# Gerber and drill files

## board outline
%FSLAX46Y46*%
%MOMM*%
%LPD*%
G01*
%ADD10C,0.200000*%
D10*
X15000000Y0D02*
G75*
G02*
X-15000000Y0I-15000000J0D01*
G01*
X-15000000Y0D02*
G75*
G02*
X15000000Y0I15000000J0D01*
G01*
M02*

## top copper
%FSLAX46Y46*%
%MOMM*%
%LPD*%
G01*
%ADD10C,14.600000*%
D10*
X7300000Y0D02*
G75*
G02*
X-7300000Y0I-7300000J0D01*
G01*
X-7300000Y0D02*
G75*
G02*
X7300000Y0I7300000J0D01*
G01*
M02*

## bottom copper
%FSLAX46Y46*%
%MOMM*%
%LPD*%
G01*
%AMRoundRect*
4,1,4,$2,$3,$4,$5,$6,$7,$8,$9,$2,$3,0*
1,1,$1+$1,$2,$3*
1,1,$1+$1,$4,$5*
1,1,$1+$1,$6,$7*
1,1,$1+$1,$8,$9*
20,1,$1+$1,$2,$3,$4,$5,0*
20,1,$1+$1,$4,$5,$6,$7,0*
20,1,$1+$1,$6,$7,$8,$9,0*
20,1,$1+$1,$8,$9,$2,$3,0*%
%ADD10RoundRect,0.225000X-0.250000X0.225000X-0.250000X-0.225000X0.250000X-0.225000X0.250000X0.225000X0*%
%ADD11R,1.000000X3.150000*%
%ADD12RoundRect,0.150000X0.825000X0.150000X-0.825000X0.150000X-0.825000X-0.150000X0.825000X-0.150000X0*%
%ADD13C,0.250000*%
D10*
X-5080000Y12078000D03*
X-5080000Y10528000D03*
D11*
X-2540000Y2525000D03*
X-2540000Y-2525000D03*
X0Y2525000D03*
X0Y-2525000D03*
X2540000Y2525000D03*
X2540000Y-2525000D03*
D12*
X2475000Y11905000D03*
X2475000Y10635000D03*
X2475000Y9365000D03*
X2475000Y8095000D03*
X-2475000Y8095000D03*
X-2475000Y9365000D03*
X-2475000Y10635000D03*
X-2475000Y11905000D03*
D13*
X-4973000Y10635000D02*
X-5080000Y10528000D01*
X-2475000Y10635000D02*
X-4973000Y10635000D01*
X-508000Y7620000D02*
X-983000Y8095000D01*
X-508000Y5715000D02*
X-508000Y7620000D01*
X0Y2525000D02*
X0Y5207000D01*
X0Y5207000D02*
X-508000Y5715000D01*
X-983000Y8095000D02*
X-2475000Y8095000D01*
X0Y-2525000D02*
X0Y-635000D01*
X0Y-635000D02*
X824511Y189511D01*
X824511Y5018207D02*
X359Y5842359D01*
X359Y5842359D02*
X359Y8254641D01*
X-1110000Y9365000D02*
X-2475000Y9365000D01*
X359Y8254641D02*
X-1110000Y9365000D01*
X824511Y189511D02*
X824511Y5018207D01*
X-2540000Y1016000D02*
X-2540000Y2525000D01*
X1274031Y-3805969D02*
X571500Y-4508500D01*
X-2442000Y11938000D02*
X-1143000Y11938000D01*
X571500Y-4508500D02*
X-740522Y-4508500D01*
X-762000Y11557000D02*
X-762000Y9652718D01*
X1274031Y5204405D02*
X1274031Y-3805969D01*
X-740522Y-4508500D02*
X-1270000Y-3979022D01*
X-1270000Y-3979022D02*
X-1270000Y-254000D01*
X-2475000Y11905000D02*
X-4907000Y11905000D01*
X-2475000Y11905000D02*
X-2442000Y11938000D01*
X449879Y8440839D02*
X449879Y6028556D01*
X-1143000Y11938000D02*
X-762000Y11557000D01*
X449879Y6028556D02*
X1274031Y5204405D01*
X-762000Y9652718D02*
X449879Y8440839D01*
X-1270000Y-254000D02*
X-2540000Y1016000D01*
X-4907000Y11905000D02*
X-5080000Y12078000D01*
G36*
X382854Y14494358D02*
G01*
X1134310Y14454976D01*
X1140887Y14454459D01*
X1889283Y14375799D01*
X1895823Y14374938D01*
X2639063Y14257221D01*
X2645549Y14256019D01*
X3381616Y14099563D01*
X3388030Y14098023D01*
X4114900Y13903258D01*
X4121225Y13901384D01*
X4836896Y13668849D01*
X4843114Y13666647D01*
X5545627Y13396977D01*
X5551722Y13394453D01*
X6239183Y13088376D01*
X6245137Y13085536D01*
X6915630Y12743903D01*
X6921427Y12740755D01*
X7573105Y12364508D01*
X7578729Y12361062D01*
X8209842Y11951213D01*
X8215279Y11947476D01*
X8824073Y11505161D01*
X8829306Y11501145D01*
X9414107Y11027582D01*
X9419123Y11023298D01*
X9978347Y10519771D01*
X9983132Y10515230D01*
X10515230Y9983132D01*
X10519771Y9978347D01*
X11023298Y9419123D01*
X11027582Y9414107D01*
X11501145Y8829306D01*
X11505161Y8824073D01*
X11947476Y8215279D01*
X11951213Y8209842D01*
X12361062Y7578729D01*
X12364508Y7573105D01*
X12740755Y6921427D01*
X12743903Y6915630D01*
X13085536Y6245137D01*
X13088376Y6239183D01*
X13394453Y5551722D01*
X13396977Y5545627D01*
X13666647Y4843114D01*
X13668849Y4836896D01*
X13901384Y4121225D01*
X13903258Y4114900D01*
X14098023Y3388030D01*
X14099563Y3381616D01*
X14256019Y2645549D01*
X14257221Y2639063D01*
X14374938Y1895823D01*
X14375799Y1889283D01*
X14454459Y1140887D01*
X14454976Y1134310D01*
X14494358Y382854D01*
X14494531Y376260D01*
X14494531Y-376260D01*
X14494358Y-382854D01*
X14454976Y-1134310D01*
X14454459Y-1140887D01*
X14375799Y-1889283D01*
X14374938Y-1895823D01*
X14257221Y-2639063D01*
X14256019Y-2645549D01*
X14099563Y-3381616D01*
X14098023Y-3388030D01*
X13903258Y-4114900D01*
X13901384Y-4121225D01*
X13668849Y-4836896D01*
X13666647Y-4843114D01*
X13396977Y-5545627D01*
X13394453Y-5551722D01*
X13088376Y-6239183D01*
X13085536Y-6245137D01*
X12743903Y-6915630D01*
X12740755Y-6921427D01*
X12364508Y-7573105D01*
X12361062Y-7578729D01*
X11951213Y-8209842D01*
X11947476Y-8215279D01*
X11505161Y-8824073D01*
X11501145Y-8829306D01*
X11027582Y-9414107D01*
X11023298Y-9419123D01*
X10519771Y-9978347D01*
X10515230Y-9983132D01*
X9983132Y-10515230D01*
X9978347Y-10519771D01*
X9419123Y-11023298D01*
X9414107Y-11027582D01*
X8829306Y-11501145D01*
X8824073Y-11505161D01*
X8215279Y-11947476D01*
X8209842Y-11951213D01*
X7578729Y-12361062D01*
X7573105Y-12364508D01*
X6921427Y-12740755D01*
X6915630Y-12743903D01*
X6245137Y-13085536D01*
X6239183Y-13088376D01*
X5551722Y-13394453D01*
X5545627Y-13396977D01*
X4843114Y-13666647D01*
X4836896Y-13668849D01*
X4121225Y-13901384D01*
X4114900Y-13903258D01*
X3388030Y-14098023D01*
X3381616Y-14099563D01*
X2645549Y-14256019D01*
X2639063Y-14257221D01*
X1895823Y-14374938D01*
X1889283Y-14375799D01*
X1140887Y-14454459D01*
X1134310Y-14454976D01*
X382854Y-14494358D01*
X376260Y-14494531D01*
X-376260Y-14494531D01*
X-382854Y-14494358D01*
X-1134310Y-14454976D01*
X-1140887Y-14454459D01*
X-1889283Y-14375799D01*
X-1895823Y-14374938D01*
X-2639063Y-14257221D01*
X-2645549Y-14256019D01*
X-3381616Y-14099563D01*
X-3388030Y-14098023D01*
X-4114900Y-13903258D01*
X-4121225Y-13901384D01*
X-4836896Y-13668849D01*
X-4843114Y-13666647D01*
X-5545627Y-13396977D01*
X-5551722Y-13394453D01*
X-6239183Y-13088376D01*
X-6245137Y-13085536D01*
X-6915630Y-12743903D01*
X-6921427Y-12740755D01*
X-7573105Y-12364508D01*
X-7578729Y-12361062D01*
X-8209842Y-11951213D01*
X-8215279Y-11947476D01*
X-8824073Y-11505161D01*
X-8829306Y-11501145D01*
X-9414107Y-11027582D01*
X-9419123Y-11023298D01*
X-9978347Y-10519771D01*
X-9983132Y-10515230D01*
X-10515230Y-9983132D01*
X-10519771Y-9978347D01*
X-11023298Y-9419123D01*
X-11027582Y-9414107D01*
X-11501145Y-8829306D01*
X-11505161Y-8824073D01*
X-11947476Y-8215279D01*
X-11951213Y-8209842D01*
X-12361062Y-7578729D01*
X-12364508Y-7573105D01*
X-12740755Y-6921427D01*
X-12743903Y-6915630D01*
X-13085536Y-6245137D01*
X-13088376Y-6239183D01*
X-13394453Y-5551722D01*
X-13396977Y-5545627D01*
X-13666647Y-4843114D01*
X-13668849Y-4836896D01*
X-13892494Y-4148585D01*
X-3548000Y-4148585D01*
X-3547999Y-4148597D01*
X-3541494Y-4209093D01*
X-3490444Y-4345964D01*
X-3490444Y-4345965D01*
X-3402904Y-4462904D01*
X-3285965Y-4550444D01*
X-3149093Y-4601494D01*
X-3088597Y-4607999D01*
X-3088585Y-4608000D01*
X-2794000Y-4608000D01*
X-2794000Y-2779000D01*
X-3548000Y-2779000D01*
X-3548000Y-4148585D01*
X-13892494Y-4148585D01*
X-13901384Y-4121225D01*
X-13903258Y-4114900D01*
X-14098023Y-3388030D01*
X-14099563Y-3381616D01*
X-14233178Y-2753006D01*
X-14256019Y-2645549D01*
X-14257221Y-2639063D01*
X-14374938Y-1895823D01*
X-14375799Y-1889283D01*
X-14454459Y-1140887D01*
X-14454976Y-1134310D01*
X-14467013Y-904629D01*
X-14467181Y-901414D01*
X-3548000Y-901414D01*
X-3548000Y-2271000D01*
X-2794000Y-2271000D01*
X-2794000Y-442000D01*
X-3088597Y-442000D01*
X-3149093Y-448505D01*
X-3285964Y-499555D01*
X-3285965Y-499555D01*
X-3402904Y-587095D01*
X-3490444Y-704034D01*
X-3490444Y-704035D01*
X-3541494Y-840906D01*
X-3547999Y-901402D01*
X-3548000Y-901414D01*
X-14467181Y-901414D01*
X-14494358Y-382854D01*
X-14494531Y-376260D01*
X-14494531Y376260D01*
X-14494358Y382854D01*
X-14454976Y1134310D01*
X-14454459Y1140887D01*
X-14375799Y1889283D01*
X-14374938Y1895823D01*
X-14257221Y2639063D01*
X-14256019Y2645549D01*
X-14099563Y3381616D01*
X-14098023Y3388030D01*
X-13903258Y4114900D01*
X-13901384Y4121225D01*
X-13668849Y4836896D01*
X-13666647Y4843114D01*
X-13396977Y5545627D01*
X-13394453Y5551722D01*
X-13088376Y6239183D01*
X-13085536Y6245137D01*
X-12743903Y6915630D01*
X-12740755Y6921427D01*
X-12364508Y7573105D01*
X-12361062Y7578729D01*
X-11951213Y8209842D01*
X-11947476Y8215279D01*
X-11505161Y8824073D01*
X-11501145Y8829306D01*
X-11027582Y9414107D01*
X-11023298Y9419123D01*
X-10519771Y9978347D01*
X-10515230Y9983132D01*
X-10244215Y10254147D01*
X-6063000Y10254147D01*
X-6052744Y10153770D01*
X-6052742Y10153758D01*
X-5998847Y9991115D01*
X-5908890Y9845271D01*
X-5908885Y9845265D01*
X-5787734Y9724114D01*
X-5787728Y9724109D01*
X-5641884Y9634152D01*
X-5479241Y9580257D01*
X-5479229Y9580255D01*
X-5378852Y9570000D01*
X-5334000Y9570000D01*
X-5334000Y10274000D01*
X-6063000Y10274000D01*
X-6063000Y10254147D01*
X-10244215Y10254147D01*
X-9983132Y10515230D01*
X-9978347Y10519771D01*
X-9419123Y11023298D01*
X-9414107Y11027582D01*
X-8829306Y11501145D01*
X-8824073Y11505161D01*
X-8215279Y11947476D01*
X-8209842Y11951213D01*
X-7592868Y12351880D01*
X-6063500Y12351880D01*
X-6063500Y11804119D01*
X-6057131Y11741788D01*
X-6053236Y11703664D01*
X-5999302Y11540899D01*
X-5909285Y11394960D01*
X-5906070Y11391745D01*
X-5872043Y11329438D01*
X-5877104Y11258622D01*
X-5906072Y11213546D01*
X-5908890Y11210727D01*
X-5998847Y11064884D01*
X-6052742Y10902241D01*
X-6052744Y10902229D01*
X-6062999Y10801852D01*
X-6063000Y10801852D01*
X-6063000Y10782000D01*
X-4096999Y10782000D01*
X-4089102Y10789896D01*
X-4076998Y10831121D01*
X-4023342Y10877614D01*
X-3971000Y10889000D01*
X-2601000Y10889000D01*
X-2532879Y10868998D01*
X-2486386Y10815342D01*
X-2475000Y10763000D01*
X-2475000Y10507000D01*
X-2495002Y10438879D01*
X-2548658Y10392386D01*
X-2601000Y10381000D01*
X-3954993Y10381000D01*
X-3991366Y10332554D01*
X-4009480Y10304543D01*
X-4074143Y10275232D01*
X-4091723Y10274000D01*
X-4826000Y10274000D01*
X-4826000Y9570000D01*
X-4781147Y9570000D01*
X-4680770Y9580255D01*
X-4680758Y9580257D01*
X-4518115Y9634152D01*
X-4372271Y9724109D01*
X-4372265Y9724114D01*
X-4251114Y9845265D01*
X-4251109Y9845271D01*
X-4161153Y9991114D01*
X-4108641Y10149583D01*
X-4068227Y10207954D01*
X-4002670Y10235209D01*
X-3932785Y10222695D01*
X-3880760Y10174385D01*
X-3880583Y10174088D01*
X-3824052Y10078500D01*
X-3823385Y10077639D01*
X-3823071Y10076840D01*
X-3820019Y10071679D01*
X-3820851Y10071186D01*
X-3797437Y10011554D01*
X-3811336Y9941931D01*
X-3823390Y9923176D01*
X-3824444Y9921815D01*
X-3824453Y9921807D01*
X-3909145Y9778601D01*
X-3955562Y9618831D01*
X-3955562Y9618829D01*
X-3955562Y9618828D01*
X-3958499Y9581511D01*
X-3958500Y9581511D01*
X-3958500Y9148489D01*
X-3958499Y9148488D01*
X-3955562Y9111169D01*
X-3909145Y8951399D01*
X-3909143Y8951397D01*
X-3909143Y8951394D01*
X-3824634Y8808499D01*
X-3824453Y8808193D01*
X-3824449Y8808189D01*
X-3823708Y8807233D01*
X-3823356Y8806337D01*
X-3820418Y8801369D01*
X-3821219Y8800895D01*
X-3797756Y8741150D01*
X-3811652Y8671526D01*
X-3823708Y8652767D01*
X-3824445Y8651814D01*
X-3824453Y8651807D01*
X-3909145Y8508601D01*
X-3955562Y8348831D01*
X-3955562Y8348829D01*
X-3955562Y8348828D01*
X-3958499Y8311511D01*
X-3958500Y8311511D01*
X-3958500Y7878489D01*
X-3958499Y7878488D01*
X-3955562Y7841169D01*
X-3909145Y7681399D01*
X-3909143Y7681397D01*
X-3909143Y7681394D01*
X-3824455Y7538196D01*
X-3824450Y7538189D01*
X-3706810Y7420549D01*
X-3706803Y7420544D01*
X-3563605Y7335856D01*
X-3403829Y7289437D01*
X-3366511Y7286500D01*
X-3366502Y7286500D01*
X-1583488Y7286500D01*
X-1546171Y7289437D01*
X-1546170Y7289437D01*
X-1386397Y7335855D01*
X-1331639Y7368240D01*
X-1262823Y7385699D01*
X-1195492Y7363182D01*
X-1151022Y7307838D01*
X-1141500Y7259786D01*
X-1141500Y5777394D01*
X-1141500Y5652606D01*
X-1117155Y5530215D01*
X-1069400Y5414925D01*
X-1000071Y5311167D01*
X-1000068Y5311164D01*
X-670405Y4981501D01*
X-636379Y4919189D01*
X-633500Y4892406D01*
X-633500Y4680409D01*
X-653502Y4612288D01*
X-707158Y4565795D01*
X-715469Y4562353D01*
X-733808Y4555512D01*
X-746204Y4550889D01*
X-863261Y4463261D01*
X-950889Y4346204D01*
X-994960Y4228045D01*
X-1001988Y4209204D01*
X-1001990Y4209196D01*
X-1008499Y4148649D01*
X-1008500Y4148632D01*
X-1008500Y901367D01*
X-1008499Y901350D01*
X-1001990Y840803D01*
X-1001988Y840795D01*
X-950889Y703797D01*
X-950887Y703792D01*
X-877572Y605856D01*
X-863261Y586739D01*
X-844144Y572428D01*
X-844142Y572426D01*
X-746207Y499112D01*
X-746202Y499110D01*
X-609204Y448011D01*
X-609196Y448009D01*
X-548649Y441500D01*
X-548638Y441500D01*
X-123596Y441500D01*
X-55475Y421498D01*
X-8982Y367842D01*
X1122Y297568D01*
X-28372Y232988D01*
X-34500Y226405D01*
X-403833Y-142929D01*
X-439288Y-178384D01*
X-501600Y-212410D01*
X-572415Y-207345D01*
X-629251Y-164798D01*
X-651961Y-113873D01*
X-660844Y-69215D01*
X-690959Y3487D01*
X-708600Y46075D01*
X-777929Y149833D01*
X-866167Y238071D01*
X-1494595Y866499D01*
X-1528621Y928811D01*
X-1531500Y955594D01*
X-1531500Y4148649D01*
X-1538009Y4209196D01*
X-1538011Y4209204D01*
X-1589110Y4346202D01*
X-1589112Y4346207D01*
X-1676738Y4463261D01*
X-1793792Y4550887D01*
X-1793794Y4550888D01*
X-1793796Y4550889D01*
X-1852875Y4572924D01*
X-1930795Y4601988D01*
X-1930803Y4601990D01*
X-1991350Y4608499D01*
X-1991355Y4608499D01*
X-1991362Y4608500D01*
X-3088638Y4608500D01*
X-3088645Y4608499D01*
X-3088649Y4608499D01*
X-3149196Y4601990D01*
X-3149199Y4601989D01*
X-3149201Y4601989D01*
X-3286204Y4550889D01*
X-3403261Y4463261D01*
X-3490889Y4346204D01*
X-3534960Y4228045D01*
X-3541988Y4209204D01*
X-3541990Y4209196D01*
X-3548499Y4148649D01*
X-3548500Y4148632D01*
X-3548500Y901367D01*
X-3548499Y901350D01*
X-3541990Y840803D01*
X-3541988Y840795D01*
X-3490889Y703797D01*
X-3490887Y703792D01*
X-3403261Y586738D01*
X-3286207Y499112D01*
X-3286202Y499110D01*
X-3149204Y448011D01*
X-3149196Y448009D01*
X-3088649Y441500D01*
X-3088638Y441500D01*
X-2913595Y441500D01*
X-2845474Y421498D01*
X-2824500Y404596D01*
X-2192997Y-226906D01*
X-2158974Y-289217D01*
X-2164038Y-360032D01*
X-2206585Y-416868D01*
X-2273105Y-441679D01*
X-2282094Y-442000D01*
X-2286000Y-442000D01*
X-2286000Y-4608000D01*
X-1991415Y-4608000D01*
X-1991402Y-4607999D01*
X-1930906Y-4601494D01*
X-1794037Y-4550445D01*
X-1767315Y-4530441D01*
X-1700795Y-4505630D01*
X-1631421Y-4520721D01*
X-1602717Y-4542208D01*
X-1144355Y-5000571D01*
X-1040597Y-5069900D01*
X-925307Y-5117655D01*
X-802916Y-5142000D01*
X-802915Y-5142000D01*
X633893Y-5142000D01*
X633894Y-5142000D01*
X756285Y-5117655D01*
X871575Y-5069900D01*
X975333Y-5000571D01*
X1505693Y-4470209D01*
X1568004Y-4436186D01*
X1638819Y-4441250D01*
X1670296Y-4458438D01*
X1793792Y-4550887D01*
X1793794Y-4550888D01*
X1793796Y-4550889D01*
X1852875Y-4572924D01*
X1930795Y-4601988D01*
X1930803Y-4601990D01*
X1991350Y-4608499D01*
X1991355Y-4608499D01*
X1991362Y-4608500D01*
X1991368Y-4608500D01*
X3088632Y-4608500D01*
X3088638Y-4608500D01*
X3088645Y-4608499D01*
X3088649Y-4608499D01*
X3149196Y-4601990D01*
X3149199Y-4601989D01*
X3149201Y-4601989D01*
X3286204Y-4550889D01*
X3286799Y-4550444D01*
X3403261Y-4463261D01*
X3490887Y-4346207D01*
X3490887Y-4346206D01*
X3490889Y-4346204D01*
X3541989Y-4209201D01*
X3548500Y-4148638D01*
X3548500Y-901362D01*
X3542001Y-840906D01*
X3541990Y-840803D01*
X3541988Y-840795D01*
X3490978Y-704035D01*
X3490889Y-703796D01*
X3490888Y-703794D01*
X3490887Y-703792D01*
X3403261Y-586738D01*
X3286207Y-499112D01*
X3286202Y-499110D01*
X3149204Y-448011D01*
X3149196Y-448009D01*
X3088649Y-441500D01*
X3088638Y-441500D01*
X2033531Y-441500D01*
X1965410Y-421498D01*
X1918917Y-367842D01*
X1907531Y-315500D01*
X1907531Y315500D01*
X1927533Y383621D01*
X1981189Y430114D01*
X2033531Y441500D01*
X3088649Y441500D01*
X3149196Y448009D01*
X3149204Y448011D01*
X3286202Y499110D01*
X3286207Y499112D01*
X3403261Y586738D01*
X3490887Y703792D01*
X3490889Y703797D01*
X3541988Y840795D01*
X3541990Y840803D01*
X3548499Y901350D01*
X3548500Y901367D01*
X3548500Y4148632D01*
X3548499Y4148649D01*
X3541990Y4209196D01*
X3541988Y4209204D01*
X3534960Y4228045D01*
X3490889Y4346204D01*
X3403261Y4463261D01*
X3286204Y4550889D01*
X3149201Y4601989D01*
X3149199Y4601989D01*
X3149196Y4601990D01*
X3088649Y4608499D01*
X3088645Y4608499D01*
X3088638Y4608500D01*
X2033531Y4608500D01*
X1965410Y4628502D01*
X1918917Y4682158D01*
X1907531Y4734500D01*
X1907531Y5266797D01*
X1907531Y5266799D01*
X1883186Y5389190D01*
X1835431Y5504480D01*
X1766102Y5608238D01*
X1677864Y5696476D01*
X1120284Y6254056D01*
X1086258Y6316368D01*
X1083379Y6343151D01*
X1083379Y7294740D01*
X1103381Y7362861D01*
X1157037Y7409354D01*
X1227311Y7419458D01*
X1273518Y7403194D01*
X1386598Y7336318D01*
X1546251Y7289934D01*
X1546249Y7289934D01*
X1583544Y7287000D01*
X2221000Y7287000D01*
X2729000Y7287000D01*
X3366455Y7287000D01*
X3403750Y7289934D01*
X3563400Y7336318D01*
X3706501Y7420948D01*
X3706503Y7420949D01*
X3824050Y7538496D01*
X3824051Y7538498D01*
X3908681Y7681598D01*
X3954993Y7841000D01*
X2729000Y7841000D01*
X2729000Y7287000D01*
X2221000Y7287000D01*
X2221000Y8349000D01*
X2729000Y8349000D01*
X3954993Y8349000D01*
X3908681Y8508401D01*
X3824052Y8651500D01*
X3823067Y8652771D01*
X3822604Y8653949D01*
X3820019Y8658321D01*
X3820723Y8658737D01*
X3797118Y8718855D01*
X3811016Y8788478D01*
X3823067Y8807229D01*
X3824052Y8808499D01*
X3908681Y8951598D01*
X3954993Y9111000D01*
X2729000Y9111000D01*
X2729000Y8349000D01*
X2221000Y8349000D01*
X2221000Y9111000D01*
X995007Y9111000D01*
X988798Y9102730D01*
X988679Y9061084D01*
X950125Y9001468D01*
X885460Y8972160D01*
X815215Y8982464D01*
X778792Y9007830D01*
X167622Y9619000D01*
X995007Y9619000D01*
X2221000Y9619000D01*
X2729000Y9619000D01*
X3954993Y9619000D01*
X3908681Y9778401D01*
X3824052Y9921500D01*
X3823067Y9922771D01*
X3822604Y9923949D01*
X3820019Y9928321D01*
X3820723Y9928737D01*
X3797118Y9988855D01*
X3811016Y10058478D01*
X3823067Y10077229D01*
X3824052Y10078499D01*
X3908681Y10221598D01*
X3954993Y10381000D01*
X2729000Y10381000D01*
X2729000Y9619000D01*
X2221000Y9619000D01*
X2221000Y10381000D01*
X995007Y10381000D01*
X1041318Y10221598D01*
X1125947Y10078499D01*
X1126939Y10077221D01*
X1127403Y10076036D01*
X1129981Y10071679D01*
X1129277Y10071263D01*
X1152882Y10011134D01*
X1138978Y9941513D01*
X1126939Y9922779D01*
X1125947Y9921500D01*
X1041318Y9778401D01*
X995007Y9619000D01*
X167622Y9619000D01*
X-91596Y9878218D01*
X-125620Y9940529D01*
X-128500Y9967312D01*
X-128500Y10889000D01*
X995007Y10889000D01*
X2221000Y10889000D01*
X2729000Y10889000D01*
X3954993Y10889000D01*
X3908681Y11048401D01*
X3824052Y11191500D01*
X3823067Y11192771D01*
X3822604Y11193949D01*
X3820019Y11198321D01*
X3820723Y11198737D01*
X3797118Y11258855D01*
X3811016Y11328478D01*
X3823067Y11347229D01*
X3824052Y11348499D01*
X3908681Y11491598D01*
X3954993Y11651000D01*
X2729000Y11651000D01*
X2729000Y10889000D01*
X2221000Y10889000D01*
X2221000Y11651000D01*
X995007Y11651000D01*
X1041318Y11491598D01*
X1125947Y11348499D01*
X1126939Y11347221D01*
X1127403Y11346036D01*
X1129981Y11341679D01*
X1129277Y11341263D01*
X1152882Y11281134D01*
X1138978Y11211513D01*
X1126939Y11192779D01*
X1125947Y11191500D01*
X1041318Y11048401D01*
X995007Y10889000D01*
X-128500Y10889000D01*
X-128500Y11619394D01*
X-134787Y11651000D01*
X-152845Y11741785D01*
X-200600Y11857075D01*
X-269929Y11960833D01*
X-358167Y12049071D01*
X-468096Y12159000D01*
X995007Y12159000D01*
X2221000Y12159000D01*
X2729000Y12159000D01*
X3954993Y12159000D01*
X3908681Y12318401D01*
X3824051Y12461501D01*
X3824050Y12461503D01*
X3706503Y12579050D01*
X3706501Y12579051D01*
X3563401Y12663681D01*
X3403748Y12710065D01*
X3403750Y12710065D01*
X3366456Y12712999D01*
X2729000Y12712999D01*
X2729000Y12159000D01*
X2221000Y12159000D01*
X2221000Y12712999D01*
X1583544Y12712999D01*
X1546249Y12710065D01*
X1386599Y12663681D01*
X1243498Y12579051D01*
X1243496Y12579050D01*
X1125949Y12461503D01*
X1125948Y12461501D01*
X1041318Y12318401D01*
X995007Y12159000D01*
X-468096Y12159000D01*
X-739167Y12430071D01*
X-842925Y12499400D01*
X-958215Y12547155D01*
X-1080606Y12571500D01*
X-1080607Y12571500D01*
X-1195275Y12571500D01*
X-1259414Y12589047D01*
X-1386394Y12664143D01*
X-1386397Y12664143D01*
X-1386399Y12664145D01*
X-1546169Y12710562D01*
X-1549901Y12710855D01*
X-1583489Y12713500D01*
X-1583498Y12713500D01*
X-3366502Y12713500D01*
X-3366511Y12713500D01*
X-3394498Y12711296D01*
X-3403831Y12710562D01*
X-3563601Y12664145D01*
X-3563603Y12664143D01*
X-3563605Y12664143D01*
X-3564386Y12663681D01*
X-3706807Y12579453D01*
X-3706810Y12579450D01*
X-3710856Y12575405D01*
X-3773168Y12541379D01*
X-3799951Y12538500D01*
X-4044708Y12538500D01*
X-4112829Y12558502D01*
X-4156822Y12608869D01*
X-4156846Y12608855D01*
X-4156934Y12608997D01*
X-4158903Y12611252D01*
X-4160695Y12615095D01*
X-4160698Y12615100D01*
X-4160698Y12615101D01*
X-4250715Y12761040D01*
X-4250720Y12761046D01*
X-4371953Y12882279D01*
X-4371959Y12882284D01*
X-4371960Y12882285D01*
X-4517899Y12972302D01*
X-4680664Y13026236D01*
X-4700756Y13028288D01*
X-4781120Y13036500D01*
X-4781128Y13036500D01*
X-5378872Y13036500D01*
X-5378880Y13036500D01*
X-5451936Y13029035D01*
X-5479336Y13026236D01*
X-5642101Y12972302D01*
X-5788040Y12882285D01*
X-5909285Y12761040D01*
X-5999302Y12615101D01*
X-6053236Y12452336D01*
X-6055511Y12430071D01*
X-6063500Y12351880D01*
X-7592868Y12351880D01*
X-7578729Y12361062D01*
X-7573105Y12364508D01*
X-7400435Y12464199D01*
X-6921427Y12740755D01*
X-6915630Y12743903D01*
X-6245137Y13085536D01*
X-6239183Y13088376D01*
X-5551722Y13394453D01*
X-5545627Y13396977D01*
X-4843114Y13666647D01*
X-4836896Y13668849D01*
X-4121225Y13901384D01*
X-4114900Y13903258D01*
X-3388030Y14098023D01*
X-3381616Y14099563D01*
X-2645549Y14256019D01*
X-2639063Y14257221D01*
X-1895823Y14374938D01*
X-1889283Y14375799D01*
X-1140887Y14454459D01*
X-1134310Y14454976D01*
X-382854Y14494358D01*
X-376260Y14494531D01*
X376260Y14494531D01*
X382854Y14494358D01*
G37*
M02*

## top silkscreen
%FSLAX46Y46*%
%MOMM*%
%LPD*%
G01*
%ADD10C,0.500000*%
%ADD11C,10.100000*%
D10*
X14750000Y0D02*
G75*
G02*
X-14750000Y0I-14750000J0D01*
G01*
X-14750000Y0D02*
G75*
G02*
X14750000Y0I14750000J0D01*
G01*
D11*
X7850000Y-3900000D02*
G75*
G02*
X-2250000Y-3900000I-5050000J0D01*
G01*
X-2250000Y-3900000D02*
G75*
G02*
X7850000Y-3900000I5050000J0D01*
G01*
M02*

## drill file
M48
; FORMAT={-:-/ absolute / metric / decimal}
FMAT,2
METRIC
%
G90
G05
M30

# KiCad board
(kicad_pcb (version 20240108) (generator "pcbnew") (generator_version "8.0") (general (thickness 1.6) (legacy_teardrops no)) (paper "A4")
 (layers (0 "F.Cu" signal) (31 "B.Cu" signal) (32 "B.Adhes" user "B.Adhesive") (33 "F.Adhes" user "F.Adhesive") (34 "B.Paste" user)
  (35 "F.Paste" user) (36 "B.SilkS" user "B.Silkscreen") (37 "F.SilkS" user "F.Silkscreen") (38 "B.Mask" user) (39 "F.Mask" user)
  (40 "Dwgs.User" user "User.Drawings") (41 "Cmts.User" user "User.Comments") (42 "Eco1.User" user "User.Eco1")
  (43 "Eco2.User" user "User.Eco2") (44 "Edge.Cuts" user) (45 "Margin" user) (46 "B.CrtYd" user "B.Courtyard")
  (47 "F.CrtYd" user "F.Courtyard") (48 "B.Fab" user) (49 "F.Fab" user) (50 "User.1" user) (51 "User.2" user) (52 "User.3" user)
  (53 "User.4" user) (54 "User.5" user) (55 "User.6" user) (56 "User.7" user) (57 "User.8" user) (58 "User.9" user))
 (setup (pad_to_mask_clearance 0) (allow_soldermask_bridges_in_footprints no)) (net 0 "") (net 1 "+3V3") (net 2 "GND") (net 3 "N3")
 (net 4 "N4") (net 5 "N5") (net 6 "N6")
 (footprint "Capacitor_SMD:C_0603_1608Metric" (layer "B.Cu") (at -5.08 -11.303 -90)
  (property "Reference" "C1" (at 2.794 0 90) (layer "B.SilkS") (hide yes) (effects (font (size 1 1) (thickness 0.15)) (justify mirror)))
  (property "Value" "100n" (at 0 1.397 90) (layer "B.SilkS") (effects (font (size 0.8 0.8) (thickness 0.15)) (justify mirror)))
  (pad "1" smd roundrect (at -0.775 0 270) (size 0.9 0.95) (layers "B.Cu" "B.Paste" "B.Mask") (roundrect_rratio 0.25) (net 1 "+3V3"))
  (pad "2" smd roundrect (at 0.775 0 270) (size 0.9 0.95) (layers "B.Cu" "B.Paste" "B.Mask") (roundrect_rratio 0.25) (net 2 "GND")))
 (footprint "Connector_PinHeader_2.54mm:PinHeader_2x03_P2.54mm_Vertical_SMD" (layer "B.Cu") (at 0 0 -90)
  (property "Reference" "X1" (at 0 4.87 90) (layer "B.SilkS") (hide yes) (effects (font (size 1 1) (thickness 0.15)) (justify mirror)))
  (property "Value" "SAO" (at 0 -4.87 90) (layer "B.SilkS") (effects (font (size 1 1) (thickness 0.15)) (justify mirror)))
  (pad "1" smd rect (at -2.525 2.54 270) (size 3.15 1) (layers "B.Cu" "B.Paste" "B.Mask") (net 1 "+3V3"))
  (pad "2" smd rect (at 2.525 2.54 270) (size 3.15 1) (layers "B.Cu" "B.Paste" "B.Mask") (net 2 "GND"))
  (pad "3" smd rect (at -2.525 0 270) (size 3.15 1) (layers "B.Cu" "B.Paste" "B.Mask") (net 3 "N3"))
  (pad "4" smd rect (at 2.525 0 270) (size 3.15 1) (layers "B.Cu" "B.Paste" "B.Mask") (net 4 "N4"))
  (pad "5" smd rect (at -2.525 -2.54 270) (size 3.15 1) (layers "B.Cu" "B.Paste" "B.Mask") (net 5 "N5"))
  (pad "6" smd rect (at 2.525 -2.54 270) (size 3.15 1) (layers "B.Cu" "B.Paste" "B.Mask") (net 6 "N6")))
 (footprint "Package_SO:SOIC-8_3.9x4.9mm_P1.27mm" (layer "B.Cu") (at 0 -10 180)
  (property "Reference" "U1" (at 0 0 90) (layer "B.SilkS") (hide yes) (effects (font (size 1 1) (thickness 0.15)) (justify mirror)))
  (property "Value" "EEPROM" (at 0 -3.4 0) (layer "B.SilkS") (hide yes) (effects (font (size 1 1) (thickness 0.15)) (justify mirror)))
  (pad "1" smd roundrect (at -2.475 1.905 180) (size 1.95 0.6) (layers "B.Cu" "B.Paste" "B.Mask") (roundrect_rratio 0.25) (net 2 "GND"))
  (pad "2" smd roundrect (at -2.475 0.635 180) (size 1.95 0.6) (layers "B.Cu" "B.Paste" "B.Mask") (roundrect_rratio 0.25) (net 2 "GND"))
  (pad "3" smd roundrect (at -2.475 -0.635 180) (size 1.95 0.6) (layers "B.Cu" "B.Paste" "B.Mask") (roundrect_rratio 0.25) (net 2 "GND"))
  (pad "4" smd roundrect (at -2.475 -1.905 180) (size 1.95 0.6) (layers "B.Cu" "B.Paste" "B.Mask") (roundrect_rratio 0.25) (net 2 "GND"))
  (pad "5" smd roundrect (at 2.475 -1.905 180) (size 1.95 0.6) (layers "B.Cu" "B.Paste" "B.Mask") (roundrect_rratio 0.25) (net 3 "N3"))
  (pad "6" smd roundrect (at 2.475 -0.635 180) (size 1.95 0.6) (layers "B.Cu" "B.Paste" "B.Mask") (roundrect_rratio 0.25) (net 4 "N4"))
  (pad "7" smd roundrect (at 2.475 0.635 180) (size 1.95 0.6) (layers "B.Cu" "B.Paste" "B.Mask") (roundrect_rratio 0.25) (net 2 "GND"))
  (pad "8" smd roundrect (at 2.475 1.905 180) (size 1.95 0.6) (layers "B.Cu" "B.Paste" "B.Mask") (roundrect_rratio 0.25) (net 1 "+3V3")))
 (gr_circle (center 0 0) (end 14.5 0) (stroke (width 0.2) (type solid)) (fill solid) (layer "F.Cu"))
 (gr_circle (center 0 0) (end 14.75 0) (stroke (width 0.5) (type solid)) (fill none) (layer "F.SilkS"))
 (gr_circle (center 2.8 3.9) (end 12.8 3.9) (stroke (width 0.2) (type solid)) (fill solid) (layer "F.SilkS"))
 (gr_circle (center 0 0) (end 15 0) (stroke (width 0.2) (type solid)) (fill none) (layer "Edge.Cuts"))
 (segment (start -4.973 -10.635) (end -5.08 -10.528) (width 0.25) (layer "B.Cu") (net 2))
 (segment (start -2.475 -10.635) (end -4.973 -10.635) (width 0.25) (layer "B.Cu") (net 2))
 (segment (start -0.508 -7.62) (end -0.983 -8.095) (width 0.25) (layer "B.Cu") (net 3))
 (segment (start -0.508 -5.715) (end -0.508 -7.62) (width 0.25) (layer "B.Cu") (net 3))
 (segment (start 0 -2.525) (end 0 -5.207) (width 0.25) (layer "B.Cu") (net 3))
 (segment (start 0 -5.207) (end -0.508 -5.715) (width 0.25) (layer "B.Cu") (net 3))
 (segment (start -0.983 -8.095) (end -2.475 -8.095) (width 0.25) (layer "B.Cu") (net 3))
 (segment (start 0 2.525) (end 0 0.635) (width 0.25) (layer "B.Cu") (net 4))
 (segment (start 0 0.635) (end 0.824511 -0.189511) (width 0.25) (layer "B.Cu") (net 4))
 (segment (start 0.824511 -5.018207) (end 0.000359 -5.842359) (width 0.25) (layer "B.Cu") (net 4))
 (segment (start 0.000359 -5.842359) (end 0.000359 -8.254641) (width 0.25) (layer "B.Cu") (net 4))
 (segment (start -1.11 -9.365) (end -2.475 -9.365) (width 0.25) (layer "B.Cu") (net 4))
 (segment (start 0.000359 -8.254641) (end -1.11 -9.365) (width 0.25) (layer "B.Cu") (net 4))
 (segment (start 0.824511 -0.189511) (end 0.824511 -5.018207) (width 0.25) (layer "B.Cu") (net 4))
 (segment (start -2.54 -1.016) (end -2.54 -2.525) (width 0.25) (layer "B.Cu") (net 1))
 (segment (start 1.274031 3.805969) (end 0.5715 4.5085) (width 0.25) (layer "B.Cu") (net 1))
 (segment (start -2.442 -11.938) (end -1.143 -11.938) (width 0.25) (layer "B.Cu") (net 1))
 (segment (start 0.5715 4.5085) (end -0.740522 4.5085) (width 0.25) (layer "B.Cu") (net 1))
 (segment (start -0.762 -11.557) (end -0.762 -9.652718) (width 0.25) (layer "B.Cu") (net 1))
 (segment (start 1.274031 -5.204405) (end 1.274031 3.805969) (width 0.25) (layer "B.Cu") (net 1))
 (segment (start -0.740522 4.5085) (end -1.27 3.979022) (width 0.25) (layer "B.Cu") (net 1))
 (segment (start -1.27 3.979022) (end -1.27 0.254) (width 0.25) (layer "B.Cu") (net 1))
 (segment (start -2.475 -11.905) (end -4.907 -11.905) (width 0.25) (layer "B.Cu") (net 1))
 (segment (start -2.475 -11.905) (end -2.442 -11.938) (width 0.25) (layer "B.Cu") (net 1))
 (segment (start 0.449879 -8.440839) (end 0.449879 -6.028556) (width 0.25) (layer "B.Cu") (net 1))
 (segment (start -1.143 -11.938) (end -0.762 -11.557) (width 0.25) (layer "B.Cu") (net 1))
 (segment (start 0.449879 -6.028556) (end 1.274031 -5.204405) (width 0.25) (layer "B.Cu") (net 1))
 (segment (start -0.762 -9.652718) (end 0.449879 -8.440839) (width 0.25) (layer "B.Cu") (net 1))
 (segment (start -1.27 0.254) (end -2.54 -1.016) (width 0.25) (layer "B.Cu") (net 1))
 (segment (start -4.907 -11.905) (end -5.08 -12.078) (width 0.25) (layer "B.Cu") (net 1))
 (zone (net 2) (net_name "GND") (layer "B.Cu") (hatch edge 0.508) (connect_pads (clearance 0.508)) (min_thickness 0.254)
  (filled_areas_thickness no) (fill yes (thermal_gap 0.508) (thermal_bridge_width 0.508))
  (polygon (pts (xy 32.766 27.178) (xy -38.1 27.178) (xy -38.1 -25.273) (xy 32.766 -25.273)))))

